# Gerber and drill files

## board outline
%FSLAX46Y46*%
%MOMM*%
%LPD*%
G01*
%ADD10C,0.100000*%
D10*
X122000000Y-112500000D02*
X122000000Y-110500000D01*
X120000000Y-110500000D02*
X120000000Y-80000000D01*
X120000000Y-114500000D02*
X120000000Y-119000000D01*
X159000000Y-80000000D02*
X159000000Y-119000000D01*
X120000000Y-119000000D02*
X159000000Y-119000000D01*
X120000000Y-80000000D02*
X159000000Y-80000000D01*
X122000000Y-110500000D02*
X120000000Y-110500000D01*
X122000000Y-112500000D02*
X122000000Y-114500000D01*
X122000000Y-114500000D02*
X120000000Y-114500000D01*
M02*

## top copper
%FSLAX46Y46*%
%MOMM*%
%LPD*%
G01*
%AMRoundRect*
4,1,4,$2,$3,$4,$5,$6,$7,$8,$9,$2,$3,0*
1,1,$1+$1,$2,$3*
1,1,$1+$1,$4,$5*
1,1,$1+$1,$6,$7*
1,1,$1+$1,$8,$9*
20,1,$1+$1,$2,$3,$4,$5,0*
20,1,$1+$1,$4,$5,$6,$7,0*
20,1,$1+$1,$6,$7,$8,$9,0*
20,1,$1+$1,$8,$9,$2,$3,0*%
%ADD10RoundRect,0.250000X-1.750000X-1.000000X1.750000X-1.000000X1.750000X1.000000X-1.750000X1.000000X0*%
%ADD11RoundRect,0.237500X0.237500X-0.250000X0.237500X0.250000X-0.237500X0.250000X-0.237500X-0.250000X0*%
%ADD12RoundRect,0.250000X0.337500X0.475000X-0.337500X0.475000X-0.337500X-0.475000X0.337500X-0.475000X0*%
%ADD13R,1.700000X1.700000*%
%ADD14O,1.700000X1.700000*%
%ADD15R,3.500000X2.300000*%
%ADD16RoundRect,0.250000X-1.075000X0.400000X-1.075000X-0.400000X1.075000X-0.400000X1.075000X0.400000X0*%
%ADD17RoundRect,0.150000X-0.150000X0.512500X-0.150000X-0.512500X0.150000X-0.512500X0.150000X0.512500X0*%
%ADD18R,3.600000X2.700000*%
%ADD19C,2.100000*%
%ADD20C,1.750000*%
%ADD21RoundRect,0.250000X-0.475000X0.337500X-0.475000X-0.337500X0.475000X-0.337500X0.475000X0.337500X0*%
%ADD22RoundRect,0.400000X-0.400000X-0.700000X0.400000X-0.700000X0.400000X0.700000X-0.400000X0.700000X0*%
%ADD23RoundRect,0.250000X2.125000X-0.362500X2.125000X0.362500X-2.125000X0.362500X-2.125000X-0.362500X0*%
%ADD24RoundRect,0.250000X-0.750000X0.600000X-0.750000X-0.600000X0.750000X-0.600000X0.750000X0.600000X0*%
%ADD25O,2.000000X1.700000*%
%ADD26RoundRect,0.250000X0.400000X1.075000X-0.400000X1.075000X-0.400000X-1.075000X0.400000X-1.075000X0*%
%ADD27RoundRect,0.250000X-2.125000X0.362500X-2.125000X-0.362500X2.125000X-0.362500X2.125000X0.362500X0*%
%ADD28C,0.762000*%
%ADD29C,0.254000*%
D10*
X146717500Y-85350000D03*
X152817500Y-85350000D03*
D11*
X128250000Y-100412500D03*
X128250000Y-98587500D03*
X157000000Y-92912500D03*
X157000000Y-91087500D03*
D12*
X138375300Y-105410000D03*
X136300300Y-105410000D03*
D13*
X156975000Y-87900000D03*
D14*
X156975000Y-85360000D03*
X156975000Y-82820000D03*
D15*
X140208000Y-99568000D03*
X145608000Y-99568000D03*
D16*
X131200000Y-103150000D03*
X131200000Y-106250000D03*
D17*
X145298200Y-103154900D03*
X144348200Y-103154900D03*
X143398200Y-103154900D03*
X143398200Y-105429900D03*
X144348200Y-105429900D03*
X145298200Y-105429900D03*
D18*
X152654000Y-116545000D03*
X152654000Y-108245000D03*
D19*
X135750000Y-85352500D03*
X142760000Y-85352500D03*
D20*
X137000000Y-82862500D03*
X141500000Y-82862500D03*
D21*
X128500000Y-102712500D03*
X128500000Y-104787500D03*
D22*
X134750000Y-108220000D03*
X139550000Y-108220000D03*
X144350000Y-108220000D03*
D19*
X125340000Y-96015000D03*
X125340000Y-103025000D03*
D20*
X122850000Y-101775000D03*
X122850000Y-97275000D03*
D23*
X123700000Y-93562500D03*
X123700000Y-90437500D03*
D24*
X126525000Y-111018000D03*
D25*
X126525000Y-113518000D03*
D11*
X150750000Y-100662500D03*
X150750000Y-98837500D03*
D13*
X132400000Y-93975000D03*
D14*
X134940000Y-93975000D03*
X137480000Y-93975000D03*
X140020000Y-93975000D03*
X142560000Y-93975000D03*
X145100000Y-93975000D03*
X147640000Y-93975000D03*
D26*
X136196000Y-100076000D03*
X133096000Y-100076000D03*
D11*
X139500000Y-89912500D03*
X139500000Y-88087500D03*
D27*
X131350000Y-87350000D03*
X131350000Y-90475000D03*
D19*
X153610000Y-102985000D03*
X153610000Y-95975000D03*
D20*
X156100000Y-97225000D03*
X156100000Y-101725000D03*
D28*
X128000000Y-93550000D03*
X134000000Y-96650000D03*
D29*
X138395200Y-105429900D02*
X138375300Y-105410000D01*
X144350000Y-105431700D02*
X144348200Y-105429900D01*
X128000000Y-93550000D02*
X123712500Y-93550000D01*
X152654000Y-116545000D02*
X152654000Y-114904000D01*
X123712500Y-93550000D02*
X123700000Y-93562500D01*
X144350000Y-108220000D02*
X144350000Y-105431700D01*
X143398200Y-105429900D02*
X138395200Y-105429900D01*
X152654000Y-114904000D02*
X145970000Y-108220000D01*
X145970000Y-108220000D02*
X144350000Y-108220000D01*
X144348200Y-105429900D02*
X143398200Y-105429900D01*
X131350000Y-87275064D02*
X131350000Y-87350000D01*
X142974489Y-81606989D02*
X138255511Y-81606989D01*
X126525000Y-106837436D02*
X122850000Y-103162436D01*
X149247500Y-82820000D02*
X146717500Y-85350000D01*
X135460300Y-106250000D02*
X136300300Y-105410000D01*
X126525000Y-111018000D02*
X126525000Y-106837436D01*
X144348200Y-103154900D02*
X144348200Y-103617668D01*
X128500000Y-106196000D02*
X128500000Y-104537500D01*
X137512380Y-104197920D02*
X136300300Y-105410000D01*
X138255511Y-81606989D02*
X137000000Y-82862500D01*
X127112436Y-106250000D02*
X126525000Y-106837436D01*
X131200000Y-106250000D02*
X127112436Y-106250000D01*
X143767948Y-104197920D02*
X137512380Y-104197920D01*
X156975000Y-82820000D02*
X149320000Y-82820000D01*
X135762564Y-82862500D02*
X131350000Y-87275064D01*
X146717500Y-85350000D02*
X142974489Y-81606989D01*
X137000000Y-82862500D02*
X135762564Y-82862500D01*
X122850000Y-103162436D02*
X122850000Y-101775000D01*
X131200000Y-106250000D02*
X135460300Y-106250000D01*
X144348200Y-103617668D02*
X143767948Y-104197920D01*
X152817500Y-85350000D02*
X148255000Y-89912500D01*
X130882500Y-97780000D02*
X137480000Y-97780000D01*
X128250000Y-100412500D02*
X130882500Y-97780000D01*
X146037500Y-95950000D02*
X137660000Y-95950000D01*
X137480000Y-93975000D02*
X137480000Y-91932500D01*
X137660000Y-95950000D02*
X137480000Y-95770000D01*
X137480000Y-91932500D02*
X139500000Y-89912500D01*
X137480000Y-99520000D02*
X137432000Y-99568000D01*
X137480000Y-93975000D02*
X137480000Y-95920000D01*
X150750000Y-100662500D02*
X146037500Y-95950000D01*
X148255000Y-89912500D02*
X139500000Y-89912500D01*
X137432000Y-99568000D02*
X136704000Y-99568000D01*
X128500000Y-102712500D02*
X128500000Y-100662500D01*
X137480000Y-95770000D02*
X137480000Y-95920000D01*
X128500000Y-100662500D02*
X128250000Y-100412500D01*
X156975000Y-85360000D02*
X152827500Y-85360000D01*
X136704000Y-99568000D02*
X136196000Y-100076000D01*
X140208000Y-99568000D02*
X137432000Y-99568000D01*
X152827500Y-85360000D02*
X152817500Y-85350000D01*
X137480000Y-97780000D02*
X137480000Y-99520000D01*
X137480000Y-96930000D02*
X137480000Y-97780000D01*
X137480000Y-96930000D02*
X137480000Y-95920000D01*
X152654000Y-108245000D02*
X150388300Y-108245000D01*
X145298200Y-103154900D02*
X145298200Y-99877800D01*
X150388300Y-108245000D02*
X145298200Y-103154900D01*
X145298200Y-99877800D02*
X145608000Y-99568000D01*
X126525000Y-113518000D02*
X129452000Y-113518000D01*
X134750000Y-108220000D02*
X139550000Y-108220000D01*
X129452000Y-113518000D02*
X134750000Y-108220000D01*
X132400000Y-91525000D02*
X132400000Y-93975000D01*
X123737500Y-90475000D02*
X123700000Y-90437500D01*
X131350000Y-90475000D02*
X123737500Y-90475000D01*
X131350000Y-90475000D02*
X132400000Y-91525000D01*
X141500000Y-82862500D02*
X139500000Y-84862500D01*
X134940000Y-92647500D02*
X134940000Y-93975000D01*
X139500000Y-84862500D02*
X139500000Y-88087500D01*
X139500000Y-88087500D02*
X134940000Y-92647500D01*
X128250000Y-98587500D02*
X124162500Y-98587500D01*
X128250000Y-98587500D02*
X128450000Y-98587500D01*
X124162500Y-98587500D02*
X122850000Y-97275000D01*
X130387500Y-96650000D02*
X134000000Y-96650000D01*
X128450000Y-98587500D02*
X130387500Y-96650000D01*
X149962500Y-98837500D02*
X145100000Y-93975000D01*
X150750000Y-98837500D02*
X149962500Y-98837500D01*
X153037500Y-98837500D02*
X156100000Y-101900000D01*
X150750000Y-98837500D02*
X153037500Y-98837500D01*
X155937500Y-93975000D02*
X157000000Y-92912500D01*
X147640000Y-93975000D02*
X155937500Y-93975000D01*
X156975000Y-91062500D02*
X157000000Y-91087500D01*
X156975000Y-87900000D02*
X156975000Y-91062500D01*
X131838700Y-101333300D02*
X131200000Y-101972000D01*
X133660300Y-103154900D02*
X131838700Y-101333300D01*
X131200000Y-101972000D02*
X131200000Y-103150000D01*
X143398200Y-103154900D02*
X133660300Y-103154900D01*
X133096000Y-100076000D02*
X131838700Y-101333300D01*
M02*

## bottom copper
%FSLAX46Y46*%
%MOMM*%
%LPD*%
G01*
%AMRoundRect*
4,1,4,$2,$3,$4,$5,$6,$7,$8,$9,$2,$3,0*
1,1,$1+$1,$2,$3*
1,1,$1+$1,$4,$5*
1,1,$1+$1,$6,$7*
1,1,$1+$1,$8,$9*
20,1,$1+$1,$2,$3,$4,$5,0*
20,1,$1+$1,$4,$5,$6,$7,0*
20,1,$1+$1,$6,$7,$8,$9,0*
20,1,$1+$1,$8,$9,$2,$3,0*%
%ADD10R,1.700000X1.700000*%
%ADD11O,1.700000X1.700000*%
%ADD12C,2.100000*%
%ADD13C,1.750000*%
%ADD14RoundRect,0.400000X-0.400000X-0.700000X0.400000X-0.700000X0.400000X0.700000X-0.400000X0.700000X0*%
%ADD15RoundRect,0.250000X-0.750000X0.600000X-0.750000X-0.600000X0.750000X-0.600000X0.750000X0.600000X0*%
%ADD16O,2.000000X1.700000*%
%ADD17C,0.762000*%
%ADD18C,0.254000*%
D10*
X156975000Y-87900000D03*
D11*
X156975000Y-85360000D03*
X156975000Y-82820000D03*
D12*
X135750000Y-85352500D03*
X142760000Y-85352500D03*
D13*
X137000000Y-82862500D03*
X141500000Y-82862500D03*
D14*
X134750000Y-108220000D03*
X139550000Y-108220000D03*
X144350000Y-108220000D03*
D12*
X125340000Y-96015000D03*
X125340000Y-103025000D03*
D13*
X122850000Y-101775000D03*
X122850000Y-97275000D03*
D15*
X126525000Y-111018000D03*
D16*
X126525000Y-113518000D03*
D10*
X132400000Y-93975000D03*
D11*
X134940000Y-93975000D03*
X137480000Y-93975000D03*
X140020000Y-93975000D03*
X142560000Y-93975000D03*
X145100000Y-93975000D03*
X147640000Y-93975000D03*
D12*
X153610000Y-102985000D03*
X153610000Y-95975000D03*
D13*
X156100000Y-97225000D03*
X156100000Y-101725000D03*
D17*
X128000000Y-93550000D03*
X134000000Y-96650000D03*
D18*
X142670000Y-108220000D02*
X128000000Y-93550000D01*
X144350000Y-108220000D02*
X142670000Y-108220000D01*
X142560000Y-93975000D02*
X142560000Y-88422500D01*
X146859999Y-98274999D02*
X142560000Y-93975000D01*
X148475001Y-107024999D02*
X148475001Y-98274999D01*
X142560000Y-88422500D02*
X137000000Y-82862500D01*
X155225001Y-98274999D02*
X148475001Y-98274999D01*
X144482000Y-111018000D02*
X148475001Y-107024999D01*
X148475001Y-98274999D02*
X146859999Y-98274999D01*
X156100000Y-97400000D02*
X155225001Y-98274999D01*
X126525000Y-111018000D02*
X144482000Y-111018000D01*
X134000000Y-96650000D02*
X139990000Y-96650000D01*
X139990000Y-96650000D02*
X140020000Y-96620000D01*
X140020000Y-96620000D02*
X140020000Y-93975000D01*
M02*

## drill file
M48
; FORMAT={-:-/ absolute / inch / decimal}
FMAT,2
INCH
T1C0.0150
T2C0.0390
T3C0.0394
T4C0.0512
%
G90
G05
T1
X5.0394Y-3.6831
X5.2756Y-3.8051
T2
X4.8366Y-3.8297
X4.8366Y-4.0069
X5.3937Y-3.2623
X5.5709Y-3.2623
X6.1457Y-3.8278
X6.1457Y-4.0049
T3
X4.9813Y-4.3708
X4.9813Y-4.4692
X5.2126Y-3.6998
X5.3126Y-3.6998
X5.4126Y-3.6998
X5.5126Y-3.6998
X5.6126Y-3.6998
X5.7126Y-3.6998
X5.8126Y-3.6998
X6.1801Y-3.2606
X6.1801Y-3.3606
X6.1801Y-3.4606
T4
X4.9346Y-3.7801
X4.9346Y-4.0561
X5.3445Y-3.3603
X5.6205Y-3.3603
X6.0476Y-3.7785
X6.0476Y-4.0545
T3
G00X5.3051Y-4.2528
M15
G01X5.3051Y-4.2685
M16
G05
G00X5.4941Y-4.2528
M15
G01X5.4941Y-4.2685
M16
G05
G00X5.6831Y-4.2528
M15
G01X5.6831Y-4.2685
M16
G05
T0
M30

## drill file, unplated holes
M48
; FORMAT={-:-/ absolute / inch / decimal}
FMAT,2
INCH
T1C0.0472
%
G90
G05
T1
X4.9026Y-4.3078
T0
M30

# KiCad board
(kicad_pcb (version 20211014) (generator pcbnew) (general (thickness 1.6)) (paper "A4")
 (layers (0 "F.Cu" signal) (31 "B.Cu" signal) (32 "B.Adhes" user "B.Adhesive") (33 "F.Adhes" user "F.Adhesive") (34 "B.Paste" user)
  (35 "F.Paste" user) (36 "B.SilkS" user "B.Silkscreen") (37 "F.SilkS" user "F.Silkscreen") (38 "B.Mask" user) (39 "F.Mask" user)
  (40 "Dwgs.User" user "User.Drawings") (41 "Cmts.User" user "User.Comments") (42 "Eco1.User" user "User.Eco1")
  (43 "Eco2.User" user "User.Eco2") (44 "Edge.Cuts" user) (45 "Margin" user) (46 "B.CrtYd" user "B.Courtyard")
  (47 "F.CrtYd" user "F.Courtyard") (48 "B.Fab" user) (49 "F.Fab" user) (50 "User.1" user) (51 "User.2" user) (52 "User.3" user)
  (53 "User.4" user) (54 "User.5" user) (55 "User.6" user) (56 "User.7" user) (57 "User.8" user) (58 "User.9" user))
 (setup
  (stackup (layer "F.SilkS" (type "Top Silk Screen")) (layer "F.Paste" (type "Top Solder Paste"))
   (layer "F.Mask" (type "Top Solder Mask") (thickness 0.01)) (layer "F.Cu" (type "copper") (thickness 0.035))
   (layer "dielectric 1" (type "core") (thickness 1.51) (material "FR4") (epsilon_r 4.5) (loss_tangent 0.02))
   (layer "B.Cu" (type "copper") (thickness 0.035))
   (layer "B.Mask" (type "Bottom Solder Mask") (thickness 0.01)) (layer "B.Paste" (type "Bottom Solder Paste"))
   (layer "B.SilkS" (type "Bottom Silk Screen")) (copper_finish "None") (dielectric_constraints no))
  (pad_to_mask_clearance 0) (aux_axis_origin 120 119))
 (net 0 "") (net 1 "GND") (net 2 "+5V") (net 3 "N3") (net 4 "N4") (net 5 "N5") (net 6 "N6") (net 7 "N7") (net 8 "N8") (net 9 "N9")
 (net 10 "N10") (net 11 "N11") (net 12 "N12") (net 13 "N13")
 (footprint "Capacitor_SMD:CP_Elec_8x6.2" (layer "F.Cu") (at 149.7675 85.35)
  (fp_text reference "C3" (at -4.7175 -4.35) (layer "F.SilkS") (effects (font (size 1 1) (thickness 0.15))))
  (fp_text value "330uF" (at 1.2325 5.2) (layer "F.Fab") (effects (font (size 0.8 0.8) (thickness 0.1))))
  (pad "1" smd roundrect locked (at -3.05 0) (size 4 2.5) (layers "F.Cu" "F.Paste" "F.Mask") (roundrect_rratio 0.1) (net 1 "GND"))
  (pad "2" smd roundrect locked (at 3.05 0) (size 4 2.5) (layers "F.Cu" "F.Paste" "F.Mask") (roundrect_rratio 0.1) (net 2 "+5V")))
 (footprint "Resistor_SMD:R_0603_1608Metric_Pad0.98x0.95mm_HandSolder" (layer "F.Cu") (at 128.25 99.5 90)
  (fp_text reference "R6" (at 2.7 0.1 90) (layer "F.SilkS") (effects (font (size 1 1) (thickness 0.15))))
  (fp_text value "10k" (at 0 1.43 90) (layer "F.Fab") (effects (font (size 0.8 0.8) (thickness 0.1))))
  (pad "1" smd roundrect locked (at -0.9125 0 90) (size 0.975 0.95) (layers "F.Cu" "F.Paste" "F.Mask") (roundrect_rratio 0.25) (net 2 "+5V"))
  (pad "2" smd roundrect locked (at 0.9125 0 90) (size 0.975 0.95) (layers "F.Cu" "F.Paste" "F.Mask") (roundrect_rratio 0.25) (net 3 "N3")))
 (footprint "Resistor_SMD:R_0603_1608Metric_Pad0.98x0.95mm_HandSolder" (layer "F.Cu") (at 157 92 90)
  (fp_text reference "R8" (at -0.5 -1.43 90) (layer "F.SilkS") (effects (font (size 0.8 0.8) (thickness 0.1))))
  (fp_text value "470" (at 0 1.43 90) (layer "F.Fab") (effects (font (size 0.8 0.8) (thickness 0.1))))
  (pad "1" smd roundrect locked (at -0.9125 0 90) (size 0.975 0.95) (layers "F.Cu" "F.Paste" "F.Mask") (roundrect_rratio 0.25) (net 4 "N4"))
  (pad "2" smd roundrect locked (at 0.9125 0 90) (size 0.975 0.95) (layers "F.Cu" "F.Paste" "F.Mask") (roundrect_rratio 0.25) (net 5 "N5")))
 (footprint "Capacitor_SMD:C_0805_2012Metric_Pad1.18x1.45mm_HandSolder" (layer "F.Cu") (at 137.3378 105.41 180)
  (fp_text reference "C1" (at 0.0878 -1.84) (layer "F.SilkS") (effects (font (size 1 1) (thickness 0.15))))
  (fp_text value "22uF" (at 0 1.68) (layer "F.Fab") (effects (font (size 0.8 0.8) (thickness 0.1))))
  (pad "1" smd roundrect locked (at -1.0375 0 180) (size 1.175 1.45) (layers "F.Cu" "F.Paste" "F.Mask") (roundrect_rratio 0.2127659574)
   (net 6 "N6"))
  (pad "2" smd roundrect locked (at 1.0375 0 180) (size 1.175 1.45) (layers "F.Cu" "F.Paste" "F.Mask") (roundrect_rratio 0.2127659574)
   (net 1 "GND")))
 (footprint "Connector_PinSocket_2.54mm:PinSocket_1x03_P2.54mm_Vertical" (layer "F.Cu") (at 156.975 87.9 180)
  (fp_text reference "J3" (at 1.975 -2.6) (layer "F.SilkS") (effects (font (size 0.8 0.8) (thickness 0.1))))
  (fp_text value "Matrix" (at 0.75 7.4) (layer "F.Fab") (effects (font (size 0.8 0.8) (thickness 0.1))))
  (pad "1" thru_hole rect locked (at 0 0 180) (size 1.7 1.7) (drill 1) (layers *.Cu *.Mask) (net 5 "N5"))
  (pad "2" thru_hole oval locked (at 0 2.54 180) (size 1.7 1.7) (drill 1) (layers *.Cu *.Mask) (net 2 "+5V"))
  (pad "3" thru_hole oval locked (at 0 5.08 180) (size 1.7 1.7) (drill 1) (layers *.Cu *.Mask) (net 1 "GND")))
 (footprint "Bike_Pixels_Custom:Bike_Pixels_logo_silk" (layer "F.Cu") (at 127.25 82.25)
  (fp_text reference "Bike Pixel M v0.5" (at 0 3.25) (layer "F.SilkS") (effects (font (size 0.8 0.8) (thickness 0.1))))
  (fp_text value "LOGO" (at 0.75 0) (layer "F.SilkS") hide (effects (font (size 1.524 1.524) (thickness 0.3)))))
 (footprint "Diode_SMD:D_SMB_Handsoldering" (layer "F.Cu") (at 142.908 99.568)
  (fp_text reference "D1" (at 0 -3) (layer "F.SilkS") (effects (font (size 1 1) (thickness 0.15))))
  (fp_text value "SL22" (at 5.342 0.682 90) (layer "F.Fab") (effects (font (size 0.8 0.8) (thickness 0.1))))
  (pad "1" smd rect locked (at -2.7 0) (size 3.5 2.3) (layers "F.Cu" "F.Paste" "F.Mask") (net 2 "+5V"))
  (pad "2" smd rect locked (at 2.7 0) (size 3.5 2.3) (layers "F.Cu" "F.Paste" "F.Mask") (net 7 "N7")))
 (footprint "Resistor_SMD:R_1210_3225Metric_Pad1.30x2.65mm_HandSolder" (layer "F.Cu") (at 131.2 104.7 -90)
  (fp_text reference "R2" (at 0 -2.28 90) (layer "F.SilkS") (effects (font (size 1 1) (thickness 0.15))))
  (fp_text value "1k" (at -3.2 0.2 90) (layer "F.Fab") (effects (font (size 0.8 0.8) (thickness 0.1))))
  (pad "1" smd roundrect locked (at -1.55 0 270) (size 1.3 2.65) (layers "F.Cu" "F.Paste" "F.Mask") (roundrect_rratio 0.1923076923)
   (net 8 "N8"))
  (pad "2" smd roundrect locked (at 1.55 0 270) (size 1.3 2.65) (layers "F.Cu" "F.Paste" "F.Mask") (roundrect_rratio 0.1923076923)
   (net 1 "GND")))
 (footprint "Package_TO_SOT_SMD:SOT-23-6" (layer "F.Cu") (at 144.3482 104.2924 -90)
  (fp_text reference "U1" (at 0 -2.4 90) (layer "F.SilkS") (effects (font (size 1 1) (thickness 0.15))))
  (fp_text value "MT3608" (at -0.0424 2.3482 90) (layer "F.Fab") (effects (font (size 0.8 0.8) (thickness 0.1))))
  (pad "1" smd roundrect locked (at -1.1375 -0.95 270) (size 1.325 0.6) (layers "F.Cu" "F.Paste" "F.Mask") (roundrect_rratio 0.25)
   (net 7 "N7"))
  (pad "2" smd roundrect locked (at -1.1375 0 270) (size 1.325 0.6) (layers "F.Cu" "F.Paste" "F.Mask") (roundrect_rratio 0.25) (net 1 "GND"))
  (pad "3" smd roundrect locked (at -1.1375 0.95 270) (size 1.325 0.6) (layers "F.Cu" "F.Paste" "F.Mask") (roundrect_rratio 0.25)
   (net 8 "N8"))
  (pad "4" smd roundrect locked (at 1.1375 0.95 270) (size 1.325 0.6) (layers "F.Cu" "F.Paste" "F.Mask") (roundrect_rratio 0.25)
   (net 6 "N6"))
  (pad "5" smd roundrect locked (at 1.1375 0 270) (size 1.325 0.6) (layers "F.Cu" "F.Paste" "F.Mask") (roundrect_rratio 0.25) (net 6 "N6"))
  (pad "6" smd roundrect locked (at 1.1375 -0.95 270) (size 1.325 0.6) (layers "F.Cu" "F.Paste" "F.Mask") (roundrect_rratio 0.25)
   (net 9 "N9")))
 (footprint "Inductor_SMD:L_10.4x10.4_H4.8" (layer "F.Cu") (at 152.654 112.395 90)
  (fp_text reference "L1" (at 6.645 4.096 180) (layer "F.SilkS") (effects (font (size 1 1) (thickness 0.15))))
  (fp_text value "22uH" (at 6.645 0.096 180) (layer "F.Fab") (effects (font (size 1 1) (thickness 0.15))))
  (pad "1" smd rect locked (at -4.15 0 90) (size 2.7 3.6) (layers "F.Cu" "F.Paste" "F.Mask") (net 6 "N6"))
  (pad "2" smd rect locked (at 4.15 0 90) (size 2.7 3.6) (layers "F.Cu" "F.Paste" "F.Mask") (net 7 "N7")))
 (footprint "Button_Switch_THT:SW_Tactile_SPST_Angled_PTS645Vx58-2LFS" (layer "F.Cu") (at 137 82.8625)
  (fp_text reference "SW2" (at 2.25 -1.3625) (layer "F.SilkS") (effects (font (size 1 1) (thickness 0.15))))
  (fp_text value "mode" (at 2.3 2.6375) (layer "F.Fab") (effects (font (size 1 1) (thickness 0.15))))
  (pad "" thru_hole circle locked (at -1.25 2.49) (size 2.1 2.1) (drill 1.3) (layers *.Cu *.Mask))
  (pad "" thru_hole circle locked (at 5.76 2.49) (size 2.1 2.1) (drill 1.3) (layers *.Cu *.Mask))
  (pad "1" thru_hole circle locked (at 0 0) (size 1.75 1.75) (drill 0.99) (layers *.Cu *.Mask) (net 1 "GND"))
  (pad "2" thru_hole circle locked (at 4.5 0) (size 1.75 1.75) (drill 0.99) (layers *.Cu *.Mask) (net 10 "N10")))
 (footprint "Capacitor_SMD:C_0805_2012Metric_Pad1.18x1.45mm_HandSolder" (layer "F.Cu") (at 128.5 103.75 -90)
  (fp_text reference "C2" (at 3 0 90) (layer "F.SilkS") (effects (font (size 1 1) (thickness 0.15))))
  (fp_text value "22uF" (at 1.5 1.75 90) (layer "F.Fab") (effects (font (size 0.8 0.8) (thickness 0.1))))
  (pad "1" smd roundrect locked (at -1.0375 0 270) (size 1.175 1.45) (layers "F.Cu" "F.Paste" "F.Mask") (roundrect_rratio 0.2127659574)
   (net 2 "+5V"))
  (pad "2" smd roundrect locked (at 1.0375 0 270) (size 1.175 1.45) (layers "F.Cu" "F.Paste" "F.Mask") (roundrect_rratio 0.2127659574)
   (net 1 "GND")))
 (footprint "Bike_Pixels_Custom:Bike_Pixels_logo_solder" (layer "F.Cu") (at 127.25 82.75)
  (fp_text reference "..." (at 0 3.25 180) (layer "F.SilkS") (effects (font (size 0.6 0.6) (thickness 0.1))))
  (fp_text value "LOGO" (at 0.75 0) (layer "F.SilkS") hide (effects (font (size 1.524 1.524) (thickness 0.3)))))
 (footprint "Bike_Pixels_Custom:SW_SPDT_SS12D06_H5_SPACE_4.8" (layer "F.Cu") (at 139.55 108.22)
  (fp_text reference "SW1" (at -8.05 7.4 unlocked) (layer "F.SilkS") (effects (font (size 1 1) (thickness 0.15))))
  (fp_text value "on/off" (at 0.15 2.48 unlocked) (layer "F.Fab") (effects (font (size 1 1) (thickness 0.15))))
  (pad "1" thru_hole roundrect (at -4.8 0) (size 1.6 2.2) (drill oval 1 1.4) (layers *.Cu *.Mask) (roundrect_rratio 0.25) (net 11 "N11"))
  (pad "2" thru_hole roundrect (at 0 0) (size 1.6 2.2) (drill oval 1 1.4) (layers *.Cu *.Mask) (roundrect_rratio 0.25) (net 11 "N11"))
  (pad "3" thru_hole roundrect (at 4.8 0) (size 1.6 2.2) (drill oval 1 1.4) (layers *.Cu *.Mask) (roundrect_rratio 0.25) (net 6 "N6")))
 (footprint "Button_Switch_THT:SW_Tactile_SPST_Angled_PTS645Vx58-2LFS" (layer "F.Cu") (at 122.85 101.775 90)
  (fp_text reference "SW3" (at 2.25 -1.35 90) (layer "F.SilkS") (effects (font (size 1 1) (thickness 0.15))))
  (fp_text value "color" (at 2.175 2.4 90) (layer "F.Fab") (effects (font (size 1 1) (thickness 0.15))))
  (pad "" thru_hole circle locked (at 5.76 2.49 90) (size 2.1 2.1) (drill 1.3) (layers *.Cu *.Mask))
  (pad "" thru_hole circle locked (at -1.25 2.49 90) (size 2.1 2.1) (drill 1.3) (layers *.Cu *.Mask))
  (pad "1" thru_hole circle locked (at 0 0 90) (size 1.75 1.75) (drill 0.99) (layers *.Cu *.Mask) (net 1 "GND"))
  (pad "2" thru_hole circle locked (at 4.5 0 90) (size 1.75 1.75) (drill 0.99) (layers *.Cu *.Mask) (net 3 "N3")))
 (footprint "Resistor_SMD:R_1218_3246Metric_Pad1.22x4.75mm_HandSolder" (layer "F.Cu") (at 123.7 92 90)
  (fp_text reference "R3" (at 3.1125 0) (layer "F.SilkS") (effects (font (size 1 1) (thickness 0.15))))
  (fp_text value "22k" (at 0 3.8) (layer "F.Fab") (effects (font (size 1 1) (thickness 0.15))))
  (pad "1" smd roundrect locked (at -1.5625 0 90) (size 1.225 4.75) (layers "F.Cu" "F.Paste" "F.Mask") (roundrect_rratio 0.2040816327)
   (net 6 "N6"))
  (pad "2" smd roundrect locked (at 1.5625 0 90) (size 1.225 4.75) (layers "F.Cu" "F.Paste" "F.Mask") (roundrect_rratio 0.2040816327)
   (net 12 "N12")))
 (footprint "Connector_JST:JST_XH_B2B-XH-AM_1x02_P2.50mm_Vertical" (layer "F.Cu") (at 126.525 111.018 -90)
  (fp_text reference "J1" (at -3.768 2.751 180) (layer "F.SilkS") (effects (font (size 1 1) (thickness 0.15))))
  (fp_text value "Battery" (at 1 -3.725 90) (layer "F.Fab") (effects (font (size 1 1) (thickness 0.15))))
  (pad "" np_thru_hole circle locked (at -1.6 2 270) (size 1.2 1.2) (drill 1.2) (layers *.Cu *.Mask))
  (pad "1" thru_hole roundrect locked (at 0 0 270) (size 1.7 2) (drill 1) (layers *.Cu *.Mask) (roundrect_rratio 0.1470588235) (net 1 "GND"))
  (pad "2" thru_hole oval locked (at 2.5 0 270) (size 1.7 2) (drill 1) (layers *.Cu *.Mask) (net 11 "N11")))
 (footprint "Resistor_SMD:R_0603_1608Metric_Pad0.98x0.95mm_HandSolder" (layer "F.Cu") (at 150.75 99.75 90)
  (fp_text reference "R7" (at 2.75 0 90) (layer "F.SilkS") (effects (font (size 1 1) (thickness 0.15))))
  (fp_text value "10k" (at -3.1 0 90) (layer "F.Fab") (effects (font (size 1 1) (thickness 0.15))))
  (pad "1" smd roundrect locked (at -0.9125 0 90) (size 0.975 0.95) (layers "F.Cu" "F.Paste" "F.Mask") (roundrect_rratio 0.25) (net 2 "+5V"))
  (pad "2" smd roundrect locked (at 0.9125 0 90) (size 0.975 0.95) (layers "F.Cu" "F.Paste" "F.Mask") (roundrect_rratio 0.25) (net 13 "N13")))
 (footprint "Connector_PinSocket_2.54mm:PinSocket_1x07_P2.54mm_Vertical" (layer "F.Cu") (at 132.4 93.975 90)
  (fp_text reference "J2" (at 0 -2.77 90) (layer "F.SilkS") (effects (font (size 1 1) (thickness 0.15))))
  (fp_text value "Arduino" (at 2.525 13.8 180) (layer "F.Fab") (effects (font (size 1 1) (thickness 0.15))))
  (pad "1" thru_hole rect locked (at 0 0 90) (size 1.7 1.7) (drill 1) (layers *.Cu *.Mask) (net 12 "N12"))
  (pad "2" thru_hole oval locked (at 0 2.54 90) (size 1.7 1.7) (drill 1) (layers *.Cu *.Mask) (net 10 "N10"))
  (pad "3" thru_hole oval locked (at 0 5.08 90) (size 1.7 1.7) (drill 1) (layers *.Cu *.Mask) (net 2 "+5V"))
  (pad "4" thru_hole oval locked (at 0 7.62 90) (size 1.7 1.7) (drill 1) (layers *.Cu *.Mask) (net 3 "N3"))
  (pad "5" thru_hole oval locked (at 0 10.16 90) (size 1.7 1.7) (drill 1) (layers *.Cu *.Mask) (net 1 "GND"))
  (pad "6" thru_hole oval locked (at 0 12.7 90) (size 1.7 1.7) (drill 1) (layers *.Cu *.Mask) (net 13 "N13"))
  (pad "7" thru_hole oval locked (at 0 15.24 90) (size 1.7 1.7) (drill 1) (layers *.Cu *.Mask) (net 4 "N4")))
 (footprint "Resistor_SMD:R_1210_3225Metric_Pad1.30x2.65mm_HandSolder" (layer "F.Cu") (at 134.646 100.076 180)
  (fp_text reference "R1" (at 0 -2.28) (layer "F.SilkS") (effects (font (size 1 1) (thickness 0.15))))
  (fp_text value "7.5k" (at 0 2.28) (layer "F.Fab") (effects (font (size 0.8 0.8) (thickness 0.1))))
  (pad "1" smd roundrect locked (at -1.55 0 180) (size 1.3 2.65) (layers "F.Cu" "F.Paste" "F.Mask") (roundrect_rratio 0.1923076923)
   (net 2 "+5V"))
  (pad "2" smd roundrect locked (at 1.55 0 180) (size 1.3 2.65) (layers "F.Cu" "F.Paste" "F.Mask") (roundrect_rratio 0.1923076923)
   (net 8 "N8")))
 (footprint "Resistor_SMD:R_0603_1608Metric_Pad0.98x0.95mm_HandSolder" (layer "F.Cu") (at 139.5 89 90)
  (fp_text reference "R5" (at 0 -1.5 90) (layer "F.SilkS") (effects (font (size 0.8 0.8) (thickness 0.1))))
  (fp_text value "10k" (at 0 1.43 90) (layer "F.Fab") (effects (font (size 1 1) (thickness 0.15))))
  (pad "1" smd roundrect locked (at -0.9125 0 90) (size 0.975 0.95) (layers "F.Cu" "F.Paste" "F.Mask") (roundrect_rratio 0.25) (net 2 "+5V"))
  (pad "2" smd roundrect locked (at 0.9125 0 90) (size 0.975 0.95) (layers "F.Cu" "F.Paste" "F.Mask") (roundrect_rratio 0.25) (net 10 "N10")))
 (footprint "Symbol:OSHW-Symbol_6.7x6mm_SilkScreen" (layer "F.Cu") (at 139.55 115.6)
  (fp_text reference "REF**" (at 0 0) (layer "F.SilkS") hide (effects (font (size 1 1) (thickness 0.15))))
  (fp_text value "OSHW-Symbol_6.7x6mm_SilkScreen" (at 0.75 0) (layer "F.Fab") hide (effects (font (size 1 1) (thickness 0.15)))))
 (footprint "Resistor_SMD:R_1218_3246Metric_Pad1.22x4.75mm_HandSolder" (layer "F.Cu") (at 131.35 88.9125 -90)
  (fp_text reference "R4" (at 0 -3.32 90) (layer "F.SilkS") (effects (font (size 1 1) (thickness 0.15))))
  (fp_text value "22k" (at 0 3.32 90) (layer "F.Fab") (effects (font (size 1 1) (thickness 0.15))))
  (pad "1" smd roundrect locked (at -1.5625 0 270) (size 1.225 4.75) (layers "F.Cu" "F.Paste" "F.Mask") (roundrect_rratio 0.2040816327)
   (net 1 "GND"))
  (pad "2" smd roundrect locked (at 1.5625 0 270) (size 1.225 4.75) (layers "F.Cu" "F.Paste" "F.Mask") (roundrect_rratio 0.2040816327)
   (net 12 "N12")))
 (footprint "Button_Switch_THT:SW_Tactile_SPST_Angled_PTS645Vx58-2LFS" (layer "F.Cu") (at 156.1 97.225 -90)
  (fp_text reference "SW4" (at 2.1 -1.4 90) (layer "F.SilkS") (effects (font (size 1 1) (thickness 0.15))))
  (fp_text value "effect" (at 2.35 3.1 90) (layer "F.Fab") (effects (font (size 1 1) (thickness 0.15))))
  (pad "" thru_hole circle locked (at 5.76 2.49 270) (size 2.1 2.1) (drill 1.3) (layers *.Cu *.Mask))
  (pad "" thru_hole circle locked (at -1.25 2.49 270) (size 2.1 2.1) (drill 1.3) (layers *.Cu *.Mask))
  (pad "1" thru_hole circle locked (at 0 0 270) (size 1.75 1.75) (drill 0.99) (layers *.Cu *.Mask) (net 1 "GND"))
  (pad "2" thru_hole circle locked (at 4.5 0 270) (size 1.75 1.75) (drill 0.99) (layers *.Cu *.Mask) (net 13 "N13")))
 (gr_line (start 122 112.5) (end 122 110.5) (layer "Edge.Cuts") (width 0.1))
 (gr_line (start 120 110.5) (end 120 80) (layer "Edge.Cuts") (width 0.1))
 (gr_line (start 120 114.5) (end 120 119) (layer "Edge.Cuts") (width 0.1))
 (gr_line (start 159 80) (end 159 119) (layer "Edge.Cuts") (width 0.1))
 (gr_line (start 120 119) (end 159 119) (layer "Edge.Cuts") (width 0.1))
 (gr_line (start 120 80) (end 159 80) (layer "Edge.Cuts") (width 0.1))
 (gr_line (start 122 110.5) (end 120 110.5) (layer "Edge.Cuts") (width 0.1))
 (gr_line (start 122 112.5) (end 122 114.5) (layer "Edge.Cuts") (width 0.1))
 (gr_line (start 122 114.5) (end 120 114.5) (layer "Edge.Cuts") (width 0.1))
 (segment (start 138.3952 105.4299) (end 138.3753 105.41) (width 0.254) (layer "F.Cu") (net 6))
 (segment (start 144.35 105.4317) (end 144.3482 105.4299) (width 0.254) (layer "F.Cu") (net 6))
 (segment (start 128 93.55) (end 123.7125 93.55) (width 0.254) (layer "F.Cu") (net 6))
 (segment (start 152.654 116.545) (end 152.654 114.904) (width 0.254) (layer "F.Cu") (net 6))
 (segment (start 123.7125 93.55) (end 123.7 93.5625) (width 0.254) (layer "F.Cu") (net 6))
 (segment (start 144.35 108.22) (end 144.35 105.4317) (width 0.254) (layer "F.Cu") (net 6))
 (segment (start 143.3982 105.4299) (end 138.3952 105.4299) (width 0.254) (layer "F.Cu") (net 6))
 (segment (start 152.654 114.904) (end 145.97 108.22) (width 0.254) (layer "F.Cu") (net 6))
 (segment (start 145.97 108.22) (end 144.35 108.22) (width 0.254) (layer "F.Cu") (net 6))
 (segment (start 144.3482 105.4299) (end 143.3982 105.4299) (width 0.254) (layer "F.Cu") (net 6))
 (via (at 128 93.55) (size 0.762) (drill 0.381) (layers "F.Cu" "B.Cu") (free) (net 6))
 (segment (start 142.67 108.22) (end 128 93.55) (width 0.254) (layer "B.Cu") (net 6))
 (segment (start 144.35 108.22) (end 142.67 108.22) (width 0.254) (layer "B.Cu") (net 6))
 (segment (start 131.35 87.275064) (end 131.35 87.35) (width 0.254) (layer "F.Cu") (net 1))
 (segment (start 142.974489 81.606989) (end 138.255511 81.606989) (width 0.254) (layer "F.Cu") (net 1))
 (segment (start 126.525 106.837436) (end 122.85 103.162436) (width 0.254) (layer "F.Cu") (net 1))
 (segment (start 149.2475 82.82) (end 146.7175 85.35) (width 0.254) (layer "F.Cu") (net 1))
 (segment (start 135.4603 106.25) (end 136.3003 105.41) (width 0.254) (layer "F.Cu") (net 1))
 (segment (start 126.525 111.018) (end 126.525 106.837436) (width 0.254) (layer "F.Cu") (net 1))
 (segment (start 144.3482 103.1549) (end 144.3482 103.617668) (width 0.254) (layer "F.Cu") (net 1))
 (segment (start 128.5 106.196) (end 128.5 104.5375) (width 0.254) (layer "F.Cu") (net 1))
 (segment (start 137.51238 104.19792) (end 136.3003 105.41) (width 0.254) (layer "F.Cu") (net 1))
 (segment (start 138.255511 81.606989) (end 137 82.8625) (width 0.254) (layer "F.Cu") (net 1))
 (segment (start 127.112436 106.25) (end 126.525 106.837436) (width 0.254) (layer "F.Cu") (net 1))
 (segment (start 131.2 106.25) (end 127.112436 106.25) (width 0.254) (layer "F.Cu") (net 1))
 (segment (start 143.767948 104.19792) (end 137.51238 104.19792) (width 0.254) (layer "F.Cu") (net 1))
 (segment (start 156.975 82.82) (end 149.32 82.82) (width 0.254) (layer "F.Cu") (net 1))
 (segment (start 135.762564 82.8625) (end 131.35 87.275064) (width 0.254) (layer "F.Cu") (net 1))
 (segment (start 146.7175 85.35) (end 142.974489 81.606989) (width 0.254) (layer "F.Cu") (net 1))
 (segment (start 137 82.8625) (end 135.762564 82.8625) (width 0.254) (layer "F.Cu") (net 1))
 (segment (start 122.85 103.162436) (end 122.85 101.775) (width 0.254) (layer "F.Cu") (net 1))
 (segment (start 131.2 106.25) (end 135.4603 106.25) (width 0.254) (layer "F.Cu") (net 1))
 (segment (start 144.3482 103.617668) (end 143.767948 104.19792) (width 0.254) (layer "F.Cu") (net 1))
 (segment (start 142.56 93.975) (end 142.56 88.4225) (width 0.254) (layer "B.Cu") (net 1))
 (segment (start 146.859999 98.274999) (end 142.56 93.975) (width 0.254) (layer "B.Cu") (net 1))
 (segment (start 148.475001 107.024999) (end 148.475001 98.274999) (width 0.254) (layer "B.Cu") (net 1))
 (segment (start 142.56 88.4225) (end 137 82.8625) (width 0.254) (layer "B.Cu") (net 1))
 (segment (start 155.225001 98.274999) (end 148.475001 98.274999) (width 0.254) (layer "B.Cu") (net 1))
 (segment (start 144.482 111.018) (end 148.475001 107.024999) (width 0.254) (layer "B.Cu") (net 1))
 (segment (start 148.475001 98.274999) (end 146.859999 98.274999) (width 0.254) (layer "B.Cu") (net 1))
 (segment (start 156.1 97.4) (end 155.225001 98.274999) (width 0.254) (layer "B.Cu") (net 1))
 (segment (start 126.525 111.018) (end 144.482 111.018) (width 0.254) (layer "B.Cu") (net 1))
 (segment (start 152.8175 85.35) (end 148.255 89.9125) (width 0.254) (layer "F.Cu") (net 2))
 (segment (start 130.8825 97.78) (end 137.48 97.78) (width 0.254) (layer "F.Cu") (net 2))
 (segment (start 128.25 100.4125) (end 130.8825 97.78) (width 0.254) (layer "F.Cu") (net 2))
 (segment (start 146.0375 95.95) (end 137.66 95.95) (width 0.254) (layer "F.Cu") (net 2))
 (segment (start 137.48 93.975) (end 137.48 91.9325) (width 0.254) (layer "F.Cu") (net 2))
 (segment (start 137.66 95.95) (end 137.48 95.77) (width 0.254) (layer "F.Cu") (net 2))
 (segment (start 137.48 91.9325) (end 139.5 89.9125) (width 0.254) (layer "F.Cu") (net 2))
 (segment (start 137.48 99.52) (end 137.432 99.568) (width 0.254) (layer "F.Cu") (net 2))
 (segment (start 137.48 93.975) (end 137.48 95.92) (width 0.254) (layer "F.Cu") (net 2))
 (segment (start 150.75 100.6625) (end 146.0375 95.95) (width 0.254) (layer "F.Cu") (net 2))
 (segment (start 148.255 89.9125) (end 139.5 89.9125) (width 0.254) (layer "F.Cu") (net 2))
 (segment (start 137.432 99.568) (end 136.704 99.568) (width 0.254) (layer "F.Cu") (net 2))
 (segment (start 128.5 102.7125) (end 128.5 100.6625) (width 0.254) (layer "F.Cu") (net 2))
 (segment (start 137.48 95.77) (end 137.48 95.92) (width 0.254) (layer "F.Cu") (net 2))
 (segment (start 128.5 100.6625) (end 128.25 100.4125) (width 0.254) (layer "F.Cu") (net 2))
 (segment (start 156.975 85.36) (end 152.8275 85.36) (width 0.254) (layer "F.Cu") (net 2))
 (segment (start 136.704 99.568) (end 136.196 100.076) (width 0.254) (layer "F.Cu") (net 2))
 (segment (start 140.208 99.568) (end 137.432 99.568) (width 0.254) (layer "F.Cu") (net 2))
 (segment (start 152.8275 85.36) (end 152.8175 85.35) (width 0.254) (layer "F.Cu") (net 2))
 (segment (start 137.48 97.78) (end 137.48 99.52) (width 0.254) (layer "F.Cu") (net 2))
 (segment (start 137.48 96.93) (end 137.48 97.78) (width 0.254) (layer "F.Cu") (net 2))
 (segment (start 137.48 96.93) (end 137.48 95.92) (width 0.254) (layer "F.Cu") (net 2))
 (segment (start 152.654 108.245) (end 150.3883 108.245) (width 0.254) (layer "F.Cu") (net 7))
 (segment (start 145.2982 103.1549) (end 145.2982 99.8778) (width 0.254) (layer "F.Cu") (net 7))
 (segment (start 150.3883 108.245) (end 145.2982 103.1549) (width 0.254) (layer "F.Cu") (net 7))
 (segment (start 145.2982 99.8778) (end 145.608 99.568) (width 0.254) (layer "F.Cu") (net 7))
 (segment (start 126.525 113.518) (end 129.452 113.518) (width 0.254) (layer "F.Cu") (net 11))
 (segment (start 134.75 108.22) (end 139.55 108.22) (width 0.254) (layer "F.Cu") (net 11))
 (segment (start 129.452 113.518) (end 134.75 108.22) (width 0.254) (layer "F.Cu") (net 11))
 (segment (start 132.4 91.525) (end 132.4 93.975) (width 0.254) (layer "F.Cu") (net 12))
 (segment (start 123.7375 90.475) (end 123.7 90.4375) (width 0.254) (layer "F.Cu") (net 12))
 (segment (start 131.35 90.475) (end 123.7375 90.475) (width 0.254) (layer "F.Cu") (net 12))
 (segment (start 131.35 90.475) (end 132.4 91.525) (width 0.254) (layer "F.Cu") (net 12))
 (segment (start 141.5 82.8625) (end 139.5 84.8625) (width 0.254) (layer "F.Cu") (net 10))
 (segment (start 134.94 92.6475) (end 134.94 93.975) (width 0.254) (layer "F.Cu") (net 10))
 (segment (start 139.5 84.8625) (end 139.5 88.0875) (width 0.254) (layer "F.Cu") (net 10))
 (segment (start 139.5 88.0875) (end 134.94 92.6475) (width 0.254) (layer "F.Cu") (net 10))
 (segment (start 128.25 98.5875) (end 124.1625 98.5875) (width 0.254) (layer "F.Cu") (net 3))
 (segment (start 128.25 98.5875) (end 128.45 98.5875) (width 0.254) (layer "F.Cu") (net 3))
 (segment (start 124.1625 98.5875) (end 122.85 97.275) (width 0.254) (layer "F.Cu") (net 3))
 (segment (start 130.3875 96.65) (end 134 96.65) (width 0.254) (layer "F.Cu") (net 3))
 (segment (start 128.45 98.5875) (end 130.3875 96.65) (width 0.254) (layer "F.Cu") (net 3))
 (via (at 134 96.65) (size 0.762) (drill 0.381) (layers "F.Cu" "B.Cu") (free) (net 3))
 (segment (start 134 96.65) (end 139.99 96.65) (width 0.254) (layer "B.Cu") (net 3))
 (segment (start 139.99 96.65) (end 140.02 96.62) (width 0.254) (layer "B.Cu") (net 3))
 (segment (start 140.02 96.62) (end 140.02 93.975) (width 0.254) (layer "B.Cu") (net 3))
 (segment (start 149.9625 98.8375) (end 145.1 93.975) (width 0.254) (layer "F.Cu") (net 13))
 (segment (start 150.75 98.8375) (end 149.9625 98.8375) (width 0.254) (layer "F.Cu") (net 13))
 (segment (start 153.0375 98.8375) (end 156.1 101.9) (width 0.254) (layer "F.Cu") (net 13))
 (segment (start 150.75 98.8375) (end 153.0375 98.8375) (width 0.254) (layer "F.Cu") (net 13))
 (segment (start 155.9375 93.975) (end 157 92.9125) (width 0.254) (layer "F.Cu") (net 4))
 (segment (start 147.64 93.975) (end 155.9375 93.975) (width 0.254) (layer "F.Cu") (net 4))
 (segment (start 156.975 91.0625) (end 157 91.0875) (width 0.254) (layer "F.Cu") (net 5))
 (segment (start 156.975 87.9) (end 156.975 91.0625) (width 0.254) (layer "F.Cu") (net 5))
 (segment (start 131.8387 101.3333) (end 131.2 101.972) (width 0.254) (layer "F.Cu") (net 8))
 (segment (start 133.6603 103.1549) (end 131.8387 101.3333) (width 0.254) (layer "F.Cu") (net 8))
 (segment (start 131.2 101.972) (end 131.2 103.15) (width 0.254) (layer "F.Cu") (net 8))
 (segment (start 143.3982 103.1549) (end 133.6603 103.1549) (width 0.254) (layer "F.Cu") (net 8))
 (segment (start 133.096 100.076) (end 131.8387 101.3333) (width 0.254) (layer "F.Cu") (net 8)))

